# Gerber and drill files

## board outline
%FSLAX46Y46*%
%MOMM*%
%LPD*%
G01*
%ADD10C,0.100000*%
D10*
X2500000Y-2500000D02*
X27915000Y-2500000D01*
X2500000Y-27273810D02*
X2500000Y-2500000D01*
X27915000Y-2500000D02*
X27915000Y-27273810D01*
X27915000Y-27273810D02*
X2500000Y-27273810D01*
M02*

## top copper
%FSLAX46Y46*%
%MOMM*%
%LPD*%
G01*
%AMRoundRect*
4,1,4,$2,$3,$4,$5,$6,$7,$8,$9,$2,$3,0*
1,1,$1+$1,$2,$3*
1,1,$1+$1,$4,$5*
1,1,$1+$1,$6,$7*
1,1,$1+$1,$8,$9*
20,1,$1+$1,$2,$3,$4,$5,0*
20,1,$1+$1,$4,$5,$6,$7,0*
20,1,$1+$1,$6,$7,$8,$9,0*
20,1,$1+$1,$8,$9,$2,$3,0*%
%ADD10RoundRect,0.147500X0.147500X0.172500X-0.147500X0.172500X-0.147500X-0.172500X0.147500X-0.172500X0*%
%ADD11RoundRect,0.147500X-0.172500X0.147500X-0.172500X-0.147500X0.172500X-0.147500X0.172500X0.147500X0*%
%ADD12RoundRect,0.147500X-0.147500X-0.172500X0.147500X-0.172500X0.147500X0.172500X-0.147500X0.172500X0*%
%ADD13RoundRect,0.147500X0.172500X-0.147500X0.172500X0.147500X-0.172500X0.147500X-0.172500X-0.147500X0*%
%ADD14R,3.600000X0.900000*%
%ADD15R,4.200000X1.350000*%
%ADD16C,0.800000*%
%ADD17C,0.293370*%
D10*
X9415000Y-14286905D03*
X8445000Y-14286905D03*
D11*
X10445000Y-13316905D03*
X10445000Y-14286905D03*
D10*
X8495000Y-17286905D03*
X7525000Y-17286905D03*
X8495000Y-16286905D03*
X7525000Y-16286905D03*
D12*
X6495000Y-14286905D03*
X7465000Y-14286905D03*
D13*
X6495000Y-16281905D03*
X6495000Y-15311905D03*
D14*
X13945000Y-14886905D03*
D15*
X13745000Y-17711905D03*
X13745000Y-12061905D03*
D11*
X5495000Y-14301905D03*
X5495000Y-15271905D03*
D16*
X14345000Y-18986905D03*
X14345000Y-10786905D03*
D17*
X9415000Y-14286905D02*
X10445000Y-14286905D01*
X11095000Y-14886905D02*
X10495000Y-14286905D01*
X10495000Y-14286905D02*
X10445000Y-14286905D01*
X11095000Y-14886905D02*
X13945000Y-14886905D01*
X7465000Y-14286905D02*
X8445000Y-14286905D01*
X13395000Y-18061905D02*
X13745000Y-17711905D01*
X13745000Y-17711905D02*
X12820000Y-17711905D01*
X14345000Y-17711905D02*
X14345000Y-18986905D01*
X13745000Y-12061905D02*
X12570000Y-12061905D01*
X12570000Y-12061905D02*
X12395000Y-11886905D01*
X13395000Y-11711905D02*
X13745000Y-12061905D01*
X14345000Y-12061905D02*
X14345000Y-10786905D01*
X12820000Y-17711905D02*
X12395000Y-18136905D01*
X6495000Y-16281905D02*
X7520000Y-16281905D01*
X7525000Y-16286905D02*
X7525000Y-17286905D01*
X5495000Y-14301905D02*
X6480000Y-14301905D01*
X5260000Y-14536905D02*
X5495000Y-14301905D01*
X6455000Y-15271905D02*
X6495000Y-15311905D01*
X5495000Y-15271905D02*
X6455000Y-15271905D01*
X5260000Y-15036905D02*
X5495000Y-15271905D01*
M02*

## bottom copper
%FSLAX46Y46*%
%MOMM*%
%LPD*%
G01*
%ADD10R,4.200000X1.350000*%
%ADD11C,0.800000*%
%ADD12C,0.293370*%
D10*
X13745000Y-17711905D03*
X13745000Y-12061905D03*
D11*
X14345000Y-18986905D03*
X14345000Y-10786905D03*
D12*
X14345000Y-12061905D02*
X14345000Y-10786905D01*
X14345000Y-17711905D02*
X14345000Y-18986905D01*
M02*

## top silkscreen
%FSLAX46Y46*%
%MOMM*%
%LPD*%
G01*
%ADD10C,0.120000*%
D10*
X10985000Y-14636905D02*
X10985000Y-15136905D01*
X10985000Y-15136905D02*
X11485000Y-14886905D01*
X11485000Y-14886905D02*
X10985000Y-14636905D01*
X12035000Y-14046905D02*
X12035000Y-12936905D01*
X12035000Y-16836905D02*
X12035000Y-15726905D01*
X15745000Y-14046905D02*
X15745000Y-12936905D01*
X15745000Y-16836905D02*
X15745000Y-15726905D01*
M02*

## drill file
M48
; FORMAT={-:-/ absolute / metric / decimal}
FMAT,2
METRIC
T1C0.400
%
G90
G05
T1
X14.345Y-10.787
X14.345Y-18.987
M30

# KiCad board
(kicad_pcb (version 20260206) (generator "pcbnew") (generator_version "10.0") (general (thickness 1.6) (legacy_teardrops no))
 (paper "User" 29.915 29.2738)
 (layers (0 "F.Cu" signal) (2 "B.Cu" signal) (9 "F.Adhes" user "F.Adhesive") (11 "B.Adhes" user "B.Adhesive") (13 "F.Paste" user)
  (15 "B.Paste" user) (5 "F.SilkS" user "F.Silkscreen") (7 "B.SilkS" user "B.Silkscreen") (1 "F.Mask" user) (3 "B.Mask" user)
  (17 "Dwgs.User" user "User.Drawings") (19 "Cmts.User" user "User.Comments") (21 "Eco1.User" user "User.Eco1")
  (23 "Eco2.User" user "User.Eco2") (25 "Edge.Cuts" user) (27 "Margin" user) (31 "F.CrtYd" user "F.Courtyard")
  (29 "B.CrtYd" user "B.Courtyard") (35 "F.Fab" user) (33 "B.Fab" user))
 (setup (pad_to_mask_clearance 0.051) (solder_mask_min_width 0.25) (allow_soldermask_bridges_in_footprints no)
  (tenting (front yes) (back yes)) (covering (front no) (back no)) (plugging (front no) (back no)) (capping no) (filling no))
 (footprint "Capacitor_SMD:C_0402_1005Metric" (layer "F.Cu") (at 8.93 14.286905 180)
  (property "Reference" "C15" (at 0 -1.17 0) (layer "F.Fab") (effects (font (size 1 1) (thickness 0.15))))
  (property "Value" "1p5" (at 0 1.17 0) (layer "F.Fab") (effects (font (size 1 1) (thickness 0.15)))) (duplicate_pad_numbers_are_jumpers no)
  (pad "1" smd roundrect (at -0.485 0 180) (size 0.59 0.64) (layers "F.Cu" "F.Mask" "F.Paste") (roundrect_rratio 0.25)
   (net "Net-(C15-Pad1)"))
  (pad "2" smd roundrect (at 0.485 0 180) (size 0.59 0.64) (layers "F.Cu" "F.Mask" "F.Paste") (roundrect_rratio 0.25) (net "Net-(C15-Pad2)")))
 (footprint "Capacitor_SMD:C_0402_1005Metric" (layer "F.Cu") (at 10.445 13.801905 -90)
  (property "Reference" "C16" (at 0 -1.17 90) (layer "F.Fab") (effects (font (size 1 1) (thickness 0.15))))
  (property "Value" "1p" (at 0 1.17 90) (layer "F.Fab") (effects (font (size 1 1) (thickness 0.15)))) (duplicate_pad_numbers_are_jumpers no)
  (pad "1" smd roundrect (at -0.485 0 270) (size 0.59 0.64) (layers "F.Cu" "F.Mask" "F.Paste") (roundrect_rratio 0.25) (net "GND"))
  (pad "2" smd roundrect (at 0.485 0 270) (size 0.59 0.64) (layers "F.Cu" "F.Mask" "F.Paste") (roundrect_rratio 0.25) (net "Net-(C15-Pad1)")))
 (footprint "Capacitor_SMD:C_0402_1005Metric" (layer "F.Cu") (at 8.01 17.286905 180)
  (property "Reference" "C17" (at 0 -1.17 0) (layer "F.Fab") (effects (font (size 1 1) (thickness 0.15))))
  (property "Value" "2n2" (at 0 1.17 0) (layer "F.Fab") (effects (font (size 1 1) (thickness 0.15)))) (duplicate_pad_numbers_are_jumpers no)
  (pad "1" smd roundrect (at -0.485 0 180) (size 0.59 0.64) (layers "F.Cu" "F.Mask" "F.Paste") (roundrect_rratio 0.25) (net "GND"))
  (pad "2" smd roundrect (at 0.485 0 180) (size 0.59 0.64) (layers "F.Cu" "F.Mask" "F.Paste") (roundrect_rratio 0.25) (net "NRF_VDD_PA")))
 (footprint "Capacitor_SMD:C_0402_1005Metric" (layer "F.Cu") (at 8.01 16.286905 180)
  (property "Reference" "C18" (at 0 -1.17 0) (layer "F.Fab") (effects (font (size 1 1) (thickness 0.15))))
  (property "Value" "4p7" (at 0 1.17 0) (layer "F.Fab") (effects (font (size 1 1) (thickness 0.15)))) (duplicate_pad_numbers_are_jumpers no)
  (pad "1" smd roundrect (at -0.485 0 180) (size 0.59 0.64) (layers "F.Cu" "F.Mask" "F.Paste") (roundrect_rratio 0.25) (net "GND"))
  (pad "2" smd roundrect (at 0.485 0 180) (size 0.59 0.64) (layers "F.Cu" "F.Mask" "F.Paste") (roundrect_rratio 0.25) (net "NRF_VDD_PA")))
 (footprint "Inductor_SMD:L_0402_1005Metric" (layer "F.Cu") (at 6.98 14.286905)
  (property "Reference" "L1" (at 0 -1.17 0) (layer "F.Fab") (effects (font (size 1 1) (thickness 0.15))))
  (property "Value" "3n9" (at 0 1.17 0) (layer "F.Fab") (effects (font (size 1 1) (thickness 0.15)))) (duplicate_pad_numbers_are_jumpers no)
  (pad "1" smd roundrect (at -0.485 0) (size 0.59 0.64) (layers "F.Cu" "F.Mask" "F.Paste") (roundrect_rratio 0.25) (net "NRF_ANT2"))
  (pad "2" smd roundrect (at 0.485 0) (size 0.59 0.64) (layers "F.Cu" "F.Mask" "F.Paste") (roundrect_rratio 0.25) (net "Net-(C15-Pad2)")))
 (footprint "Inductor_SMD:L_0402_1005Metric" (layer "F.Cu") (at 6.495 15.796905 90)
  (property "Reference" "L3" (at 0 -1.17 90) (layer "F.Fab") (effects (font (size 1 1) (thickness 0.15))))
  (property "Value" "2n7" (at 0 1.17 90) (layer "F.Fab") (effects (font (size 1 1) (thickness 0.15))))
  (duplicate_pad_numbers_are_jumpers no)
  (pad "1" smd roundrect (at -0.485 0 90) (size 0.59 0.64) (layers "F.Cu" "F.Mask" "F.Paste") (roundrect_rratio 0.25) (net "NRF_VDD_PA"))
  (pad "2" smd roundrect (at 0.485 0 90) (size 0.59 0.64) (layers "F.Cu" "F.Mask" "F.Paste") (roundrect_rratio 0.25) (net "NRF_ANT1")))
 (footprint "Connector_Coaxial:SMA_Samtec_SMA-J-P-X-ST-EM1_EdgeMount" (layer "F.Cu") (at 13.745 14.886905 90)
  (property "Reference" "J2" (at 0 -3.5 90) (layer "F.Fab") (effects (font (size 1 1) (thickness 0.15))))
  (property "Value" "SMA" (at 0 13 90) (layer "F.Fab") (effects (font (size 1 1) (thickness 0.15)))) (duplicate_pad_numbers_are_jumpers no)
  (fp_line (start 0.25 -2.76) (end -0.25 -2.76) (stroke (width 0.12) (type solid)) (layer "F.SilkS"))
  (fp_line (start -0.25 -2.76) (end 0 -2.26) (stroke (width 0.12) (type solid)) (layer "F.SilkS"))
  (fp_line (start 0 -2.26) (end 0.25 -2.76) (stroke (width 0.12) (type solid)) (layer "F.SilkS"))
  (fp_line (start 0.84 -1.71) (end 1.95 -1.71) (stroke (width 0.12) (type solid)) (layer "F.SilkS"))
  (fp_line (start -1.95 -1.71) (end -0.84 -1.71) (stroke (width 0.12) (type solid)) (layer "F.SilkS"))
  (fp_line (start 0.84 2) (end 1.95 2) (stroke (width 0.12) (type solid)) (layer "F.SilkS"))
  (fp_line (start -1.95 2) (end -0.84 2) (stroke (width 0.12) (type solid)) (layer "F.SilkS"))
  (pad "1" smd rect (at 0 0.2 90) (size 0.9 3.6) (layers "F.Cu" "F.Mask" "F.Paste") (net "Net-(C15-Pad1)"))
  (pad "2" smd rect (at -2.825 0 90) (size 1.35 4.2) (layers "F.Cu" "F.Mask" "F.Paste") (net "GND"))
  (pad "2" smd rect (at -2.825 0 90) (size 1.35 4.2) (layers "B.Cu" "B.Mask" "B.Paste") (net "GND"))
  (pad "2" smd rect (at 2.825 0 90) (size 1.35 4.2) (layers "F.Cu" "F.Mask" "F.Paste") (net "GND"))
  (pad "2" smd rect (at 2.825 0 90) (size 1.35 4.2) (layers "B.Cu" "B.Mask" "B.Paste") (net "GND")))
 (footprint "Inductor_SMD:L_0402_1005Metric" (layer "F.Cu") (at 5.495 14.786905 -90)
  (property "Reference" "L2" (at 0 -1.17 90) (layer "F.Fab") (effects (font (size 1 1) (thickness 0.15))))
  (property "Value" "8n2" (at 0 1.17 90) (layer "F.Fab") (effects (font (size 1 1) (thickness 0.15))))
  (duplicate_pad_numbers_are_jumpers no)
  (pad "1" smd roundrect (at -0.485 0 270) (size 0.59 0.64) (layers "F.Cu" "F.Mask" "F.Paste") (roundrect_rratio 0.25) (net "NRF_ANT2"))
  (pad "2" smd roundrect (at 0.485 0 270) (size 0.59 0.64) (layers "F.Cu" "F.Mask" "F.Paste") (roundrect_rratio 0.25) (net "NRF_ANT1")))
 (gr_line (start 2.5 2.5) (end 27.915 2.5) (stroke (width 0.1) (type default)) (layer "Edge.Cuts"))
 (gr_line (start 2.5 27.27381) (end 2.5 2.5) (stroke (width 0.1) (type default)) (layer "Edge.Cuts"))
 (gr_line (start 27.915 2.5) (end 27.915 27.27381) (stroke (width 0.1) (type default)) (layer "Edge.Cuts"))
 (gr_line (start 27.915 27.27381) (end 2.5 27.27381) (stroke (width 0.1) (type default)) (layer "Edge.Cuts"))
 (segment (start 9.415 14.286905) (end 10.445 14.286905) (width 0.29337) (layer "F.Cu") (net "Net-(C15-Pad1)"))
 (segment (start 11.095 14.886905) (end 10.495 14.286905) (width 0.29337) (layer "F.Cu") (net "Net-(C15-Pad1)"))
 (segment (start 10.495 14.286905) (end 10.445 14.286905) (width 0.29337) (layer "F.Cu") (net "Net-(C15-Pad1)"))
 (segment (start 11.095 14.886905) (end 13.945 14.886905) (width 0.29337) (layer "F.Cu") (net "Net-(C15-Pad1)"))
 (segment (start 7.465 14.286905) (end 8.445 14.286905) (width 0.29337) (layer "F.Cu") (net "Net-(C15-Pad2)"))
 (segment (start 13.395 18.061905) (end 13.745 17.711905) (width 0.29337) (layer "F.Cu") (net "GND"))
 (segment (start 13.745 17.711905) (end 12.82 17.711905) (width 0.29337) (layer "F.Cu") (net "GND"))
 (segment (start 14.345 17.711905) (end 14.345 18.986905) (width 0.29337) (layer "F.Cu") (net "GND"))
 (segment (start 13.745 12.061905) (end 12.57 12.061905) (width 0.29337) (layer "F.Cu") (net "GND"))
 (segment (start 12.57 12.061905) (end 12.395 11.886905) (width 0.29337) (layer "F.Cu") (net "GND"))
 (segment (start 13.395 11.711905) (end 13.745 12.061905) (width 0.29337) (layer "F.Cu") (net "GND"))
 (segment (start 14.345 12.061905) (end 14.345 10.786905) (width 0.29337) (layer "F.Cu") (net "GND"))
 (segment (start 12.82 17.711905) (end 12.395 18.136905) (width 0.29337) (layer "F.Cu") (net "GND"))
 (via (at 14.345 18.986905) (size 0.8) (drill 0.4) (layers "F.Cu" "B.Cu") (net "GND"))
 (via (at 14.345 10.786905) (size 0.8) (drill 0.4) (layers "F.Cu" "B.Cu") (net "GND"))
 (segment (start 14.345 12.061905) (end 14.345 10.786905) (width 0.29337) (layer "B.Cu") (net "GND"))
 (segment (start 14.345 17.711905) (end 14.345 18.986905) (width 0.29337) (layer "B.Cu") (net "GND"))
 (segment (start 6.495 16.281905) (end 7.52 16.281905) (width 0.29337) (layer "F.Cu") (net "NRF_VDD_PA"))
 (segment (start 7.525 16.286905) (end 7.525 17.286905) (width 0.29337) (layer "F.Cu") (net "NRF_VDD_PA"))
 (segment (start 5.495 14.301905) (end 6.48 14.301905) (width 0.29337) (layer "F.Cu") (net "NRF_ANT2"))
 (segment (start 5.26 14.536905) (end 5.495 14.301905) (width 0.29337) (layer "F.Cu") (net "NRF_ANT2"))
 (segment (start 6.455 15.271905) (end 6.495 15.311905) (width 0.29337) (layer "F.Cu") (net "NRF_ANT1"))
 (segment (start 5.495 15.271905) (end 6.455 15.271905) (width 0.29337) (layer "F.Cu") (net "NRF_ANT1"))
 (segment (start 5.26 15.036905) (end 5.495 15.271905) (width 0.29337) (layer "F.Cu") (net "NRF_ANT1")))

